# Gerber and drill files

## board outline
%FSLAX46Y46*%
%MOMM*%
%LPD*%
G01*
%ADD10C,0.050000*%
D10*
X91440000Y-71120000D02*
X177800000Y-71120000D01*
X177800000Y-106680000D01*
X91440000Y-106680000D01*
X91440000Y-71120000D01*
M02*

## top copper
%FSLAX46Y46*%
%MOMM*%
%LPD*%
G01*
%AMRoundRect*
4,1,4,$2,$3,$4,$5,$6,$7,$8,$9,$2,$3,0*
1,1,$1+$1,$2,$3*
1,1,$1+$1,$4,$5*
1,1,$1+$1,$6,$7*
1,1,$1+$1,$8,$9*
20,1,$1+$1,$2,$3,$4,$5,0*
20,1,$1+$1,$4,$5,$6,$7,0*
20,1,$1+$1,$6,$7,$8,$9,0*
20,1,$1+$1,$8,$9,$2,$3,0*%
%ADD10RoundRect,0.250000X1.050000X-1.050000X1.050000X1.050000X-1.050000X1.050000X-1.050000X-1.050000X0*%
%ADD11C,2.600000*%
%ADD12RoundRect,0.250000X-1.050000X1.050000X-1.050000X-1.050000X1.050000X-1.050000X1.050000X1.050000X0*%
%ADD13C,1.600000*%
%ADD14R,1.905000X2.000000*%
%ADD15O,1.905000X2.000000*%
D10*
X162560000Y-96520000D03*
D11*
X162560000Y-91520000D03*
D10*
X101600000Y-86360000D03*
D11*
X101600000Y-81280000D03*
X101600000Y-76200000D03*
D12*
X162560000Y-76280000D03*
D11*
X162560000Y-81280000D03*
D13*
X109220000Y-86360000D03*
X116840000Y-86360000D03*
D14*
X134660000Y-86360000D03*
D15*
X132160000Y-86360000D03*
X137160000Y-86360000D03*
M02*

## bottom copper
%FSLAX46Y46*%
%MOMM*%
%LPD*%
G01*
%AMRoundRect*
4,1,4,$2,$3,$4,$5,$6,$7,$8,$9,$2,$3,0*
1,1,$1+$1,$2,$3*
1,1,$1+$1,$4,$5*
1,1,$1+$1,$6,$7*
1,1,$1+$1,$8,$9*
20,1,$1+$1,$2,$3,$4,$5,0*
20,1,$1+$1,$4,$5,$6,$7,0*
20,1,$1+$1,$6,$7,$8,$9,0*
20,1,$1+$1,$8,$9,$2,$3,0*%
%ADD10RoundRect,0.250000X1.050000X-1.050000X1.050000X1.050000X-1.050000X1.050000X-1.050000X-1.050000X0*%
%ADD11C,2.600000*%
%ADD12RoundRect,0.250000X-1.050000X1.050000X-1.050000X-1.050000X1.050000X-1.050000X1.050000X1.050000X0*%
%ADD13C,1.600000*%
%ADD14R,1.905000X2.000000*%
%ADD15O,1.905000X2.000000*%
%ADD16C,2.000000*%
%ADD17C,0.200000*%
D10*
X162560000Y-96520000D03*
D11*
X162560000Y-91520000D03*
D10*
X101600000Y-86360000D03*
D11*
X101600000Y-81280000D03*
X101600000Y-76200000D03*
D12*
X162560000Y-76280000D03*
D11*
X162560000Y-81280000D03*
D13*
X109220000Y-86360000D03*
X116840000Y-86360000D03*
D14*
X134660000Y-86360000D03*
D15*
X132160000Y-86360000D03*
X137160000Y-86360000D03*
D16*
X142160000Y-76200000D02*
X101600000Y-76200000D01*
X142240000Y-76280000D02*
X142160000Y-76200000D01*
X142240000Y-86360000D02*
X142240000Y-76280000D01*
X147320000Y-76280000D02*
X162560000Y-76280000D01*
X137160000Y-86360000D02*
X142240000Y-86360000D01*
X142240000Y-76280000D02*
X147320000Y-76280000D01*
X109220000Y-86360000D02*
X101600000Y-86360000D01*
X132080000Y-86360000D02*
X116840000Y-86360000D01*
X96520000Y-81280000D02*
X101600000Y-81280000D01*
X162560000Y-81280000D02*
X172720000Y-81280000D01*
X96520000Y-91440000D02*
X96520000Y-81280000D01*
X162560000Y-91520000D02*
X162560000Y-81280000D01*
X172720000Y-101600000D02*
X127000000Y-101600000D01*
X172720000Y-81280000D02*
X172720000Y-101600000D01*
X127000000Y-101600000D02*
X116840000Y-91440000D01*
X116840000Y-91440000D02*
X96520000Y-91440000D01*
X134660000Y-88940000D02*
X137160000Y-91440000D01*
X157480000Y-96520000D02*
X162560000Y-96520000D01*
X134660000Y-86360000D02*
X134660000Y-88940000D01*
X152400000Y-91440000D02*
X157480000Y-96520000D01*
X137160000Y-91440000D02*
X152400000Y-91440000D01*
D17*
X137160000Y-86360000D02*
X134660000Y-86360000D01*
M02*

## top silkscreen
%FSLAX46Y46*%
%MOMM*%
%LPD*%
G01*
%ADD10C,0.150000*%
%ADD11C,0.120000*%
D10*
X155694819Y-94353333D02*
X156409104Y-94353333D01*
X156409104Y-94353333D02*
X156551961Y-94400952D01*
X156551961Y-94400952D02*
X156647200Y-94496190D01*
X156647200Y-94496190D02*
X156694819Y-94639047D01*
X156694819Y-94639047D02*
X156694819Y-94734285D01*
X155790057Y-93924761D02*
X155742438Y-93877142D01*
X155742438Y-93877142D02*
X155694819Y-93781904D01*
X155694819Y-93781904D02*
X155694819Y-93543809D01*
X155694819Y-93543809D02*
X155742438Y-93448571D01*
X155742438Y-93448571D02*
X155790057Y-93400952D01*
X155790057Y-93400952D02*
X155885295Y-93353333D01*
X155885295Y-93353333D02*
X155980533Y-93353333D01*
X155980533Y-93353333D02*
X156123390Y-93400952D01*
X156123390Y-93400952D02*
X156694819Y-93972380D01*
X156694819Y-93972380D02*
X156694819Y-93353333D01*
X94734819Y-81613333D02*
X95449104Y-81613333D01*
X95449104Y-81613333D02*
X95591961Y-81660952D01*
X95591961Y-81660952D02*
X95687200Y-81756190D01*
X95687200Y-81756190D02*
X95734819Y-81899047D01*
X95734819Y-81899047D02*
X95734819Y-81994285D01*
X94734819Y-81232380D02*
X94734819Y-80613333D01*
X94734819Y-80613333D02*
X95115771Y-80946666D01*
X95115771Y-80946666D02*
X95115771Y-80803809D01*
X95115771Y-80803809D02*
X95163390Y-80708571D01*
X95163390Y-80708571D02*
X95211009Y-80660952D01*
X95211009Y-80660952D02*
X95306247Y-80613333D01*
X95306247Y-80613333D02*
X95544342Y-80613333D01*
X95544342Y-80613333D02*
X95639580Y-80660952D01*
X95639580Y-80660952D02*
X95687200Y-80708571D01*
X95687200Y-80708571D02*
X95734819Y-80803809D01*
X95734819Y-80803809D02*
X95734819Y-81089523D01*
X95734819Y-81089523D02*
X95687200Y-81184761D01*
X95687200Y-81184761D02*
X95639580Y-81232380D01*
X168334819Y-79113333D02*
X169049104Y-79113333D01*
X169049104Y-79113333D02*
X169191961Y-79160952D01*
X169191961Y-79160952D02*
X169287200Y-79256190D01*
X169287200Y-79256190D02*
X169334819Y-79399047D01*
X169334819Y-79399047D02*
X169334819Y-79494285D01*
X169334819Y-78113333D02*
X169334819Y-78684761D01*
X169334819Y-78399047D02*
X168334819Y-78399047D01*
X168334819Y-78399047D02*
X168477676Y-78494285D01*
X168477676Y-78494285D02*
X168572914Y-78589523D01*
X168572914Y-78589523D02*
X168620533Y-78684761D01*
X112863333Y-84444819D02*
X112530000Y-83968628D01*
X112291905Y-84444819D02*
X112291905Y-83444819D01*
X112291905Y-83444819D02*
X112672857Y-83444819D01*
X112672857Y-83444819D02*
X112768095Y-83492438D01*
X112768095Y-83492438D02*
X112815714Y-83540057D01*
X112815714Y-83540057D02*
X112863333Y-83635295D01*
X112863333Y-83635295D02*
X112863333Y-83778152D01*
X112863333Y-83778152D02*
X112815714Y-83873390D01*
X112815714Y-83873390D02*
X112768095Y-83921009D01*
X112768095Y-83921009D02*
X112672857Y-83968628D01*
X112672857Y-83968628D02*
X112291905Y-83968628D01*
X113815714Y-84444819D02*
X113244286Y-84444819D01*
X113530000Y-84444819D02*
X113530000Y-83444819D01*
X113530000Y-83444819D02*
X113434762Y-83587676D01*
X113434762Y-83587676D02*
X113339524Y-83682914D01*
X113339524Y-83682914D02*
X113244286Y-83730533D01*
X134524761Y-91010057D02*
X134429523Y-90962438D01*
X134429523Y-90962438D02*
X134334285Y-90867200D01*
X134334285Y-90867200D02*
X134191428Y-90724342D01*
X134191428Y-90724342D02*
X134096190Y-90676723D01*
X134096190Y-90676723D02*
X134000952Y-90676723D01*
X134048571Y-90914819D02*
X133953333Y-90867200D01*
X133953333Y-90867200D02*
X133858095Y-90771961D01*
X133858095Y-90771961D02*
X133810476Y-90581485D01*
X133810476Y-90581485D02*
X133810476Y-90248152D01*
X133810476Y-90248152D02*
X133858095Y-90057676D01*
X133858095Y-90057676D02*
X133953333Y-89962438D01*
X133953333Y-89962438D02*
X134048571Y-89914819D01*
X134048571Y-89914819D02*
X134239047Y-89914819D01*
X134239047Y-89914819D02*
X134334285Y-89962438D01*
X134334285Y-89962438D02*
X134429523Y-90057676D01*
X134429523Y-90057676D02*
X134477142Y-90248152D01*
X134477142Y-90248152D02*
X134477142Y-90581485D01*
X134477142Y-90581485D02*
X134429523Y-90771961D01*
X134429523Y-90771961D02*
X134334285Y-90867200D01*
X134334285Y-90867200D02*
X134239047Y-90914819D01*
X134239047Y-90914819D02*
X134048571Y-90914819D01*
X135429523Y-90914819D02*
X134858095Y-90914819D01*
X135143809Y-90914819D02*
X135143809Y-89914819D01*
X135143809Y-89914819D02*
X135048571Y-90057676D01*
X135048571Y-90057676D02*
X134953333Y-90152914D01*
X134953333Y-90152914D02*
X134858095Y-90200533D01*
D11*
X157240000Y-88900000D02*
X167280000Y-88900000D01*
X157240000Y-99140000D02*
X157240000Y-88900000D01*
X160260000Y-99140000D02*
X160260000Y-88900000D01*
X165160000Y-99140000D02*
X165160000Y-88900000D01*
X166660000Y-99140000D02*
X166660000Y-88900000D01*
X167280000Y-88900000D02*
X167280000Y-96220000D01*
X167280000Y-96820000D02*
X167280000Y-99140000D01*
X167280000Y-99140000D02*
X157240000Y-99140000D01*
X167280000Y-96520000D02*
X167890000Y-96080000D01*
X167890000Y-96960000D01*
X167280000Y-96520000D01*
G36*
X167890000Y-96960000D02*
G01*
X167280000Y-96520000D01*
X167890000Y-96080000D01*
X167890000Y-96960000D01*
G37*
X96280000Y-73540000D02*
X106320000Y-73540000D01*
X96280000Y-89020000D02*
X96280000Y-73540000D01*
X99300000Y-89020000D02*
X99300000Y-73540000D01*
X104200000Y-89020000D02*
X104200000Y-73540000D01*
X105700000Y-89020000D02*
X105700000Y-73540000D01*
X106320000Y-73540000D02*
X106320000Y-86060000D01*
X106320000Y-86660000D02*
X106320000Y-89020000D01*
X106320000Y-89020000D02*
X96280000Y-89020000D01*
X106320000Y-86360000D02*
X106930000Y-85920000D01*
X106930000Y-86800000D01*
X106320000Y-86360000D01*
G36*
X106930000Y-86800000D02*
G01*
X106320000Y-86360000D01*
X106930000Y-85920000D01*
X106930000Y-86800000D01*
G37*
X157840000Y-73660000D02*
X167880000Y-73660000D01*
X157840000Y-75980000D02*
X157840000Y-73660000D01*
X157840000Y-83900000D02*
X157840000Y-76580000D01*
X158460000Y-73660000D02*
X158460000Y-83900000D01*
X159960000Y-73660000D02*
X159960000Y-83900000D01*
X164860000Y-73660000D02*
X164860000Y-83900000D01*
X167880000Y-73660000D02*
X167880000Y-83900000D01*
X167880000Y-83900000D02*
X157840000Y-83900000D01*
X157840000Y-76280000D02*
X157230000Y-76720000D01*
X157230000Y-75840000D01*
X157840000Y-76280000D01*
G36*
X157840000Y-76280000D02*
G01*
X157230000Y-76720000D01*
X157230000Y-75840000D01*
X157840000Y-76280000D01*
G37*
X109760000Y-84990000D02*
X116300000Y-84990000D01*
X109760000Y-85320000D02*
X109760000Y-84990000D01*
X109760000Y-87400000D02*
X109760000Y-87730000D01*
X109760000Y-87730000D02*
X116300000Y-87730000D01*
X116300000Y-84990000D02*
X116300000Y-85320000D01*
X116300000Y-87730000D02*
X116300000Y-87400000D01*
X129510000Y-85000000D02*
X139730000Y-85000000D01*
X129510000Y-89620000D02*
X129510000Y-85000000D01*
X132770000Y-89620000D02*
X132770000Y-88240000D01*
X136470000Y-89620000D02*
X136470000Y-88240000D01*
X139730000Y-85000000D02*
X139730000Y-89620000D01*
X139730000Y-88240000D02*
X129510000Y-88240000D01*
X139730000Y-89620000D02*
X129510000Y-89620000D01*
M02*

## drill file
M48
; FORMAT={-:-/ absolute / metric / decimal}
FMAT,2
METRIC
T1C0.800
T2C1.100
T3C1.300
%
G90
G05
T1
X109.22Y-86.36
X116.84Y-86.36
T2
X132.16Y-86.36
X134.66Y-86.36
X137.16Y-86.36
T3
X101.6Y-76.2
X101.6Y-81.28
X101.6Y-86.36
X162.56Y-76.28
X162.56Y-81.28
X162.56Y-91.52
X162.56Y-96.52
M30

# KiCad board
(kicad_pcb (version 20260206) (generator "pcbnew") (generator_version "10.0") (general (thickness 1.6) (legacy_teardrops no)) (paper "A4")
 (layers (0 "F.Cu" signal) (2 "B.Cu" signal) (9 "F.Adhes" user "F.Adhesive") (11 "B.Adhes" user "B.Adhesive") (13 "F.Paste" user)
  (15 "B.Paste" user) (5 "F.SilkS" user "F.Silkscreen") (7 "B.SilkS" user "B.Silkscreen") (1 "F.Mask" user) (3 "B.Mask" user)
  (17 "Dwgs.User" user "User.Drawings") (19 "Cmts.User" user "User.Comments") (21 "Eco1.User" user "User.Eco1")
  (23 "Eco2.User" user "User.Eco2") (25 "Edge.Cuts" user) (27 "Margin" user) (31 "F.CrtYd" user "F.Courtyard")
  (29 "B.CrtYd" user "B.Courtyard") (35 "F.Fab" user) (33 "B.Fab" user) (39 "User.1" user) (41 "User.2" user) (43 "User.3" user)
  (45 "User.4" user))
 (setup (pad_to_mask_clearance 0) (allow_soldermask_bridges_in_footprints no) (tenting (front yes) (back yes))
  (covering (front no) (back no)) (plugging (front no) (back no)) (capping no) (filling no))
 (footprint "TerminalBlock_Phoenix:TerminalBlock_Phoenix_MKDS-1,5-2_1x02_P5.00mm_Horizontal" (layer "F.Cu") (at 162.56 96.52 90)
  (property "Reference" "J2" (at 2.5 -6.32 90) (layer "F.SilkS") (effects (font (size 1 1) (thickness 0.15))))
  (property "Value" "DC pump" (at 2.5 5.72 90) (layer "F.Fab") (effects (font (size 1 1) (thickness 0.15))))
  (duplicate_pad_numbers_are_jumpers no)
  (fp_line (start 7.62 -5.32) (end 7.62 4.72) (stroke (width 0.12) (type solid)) (layer "F.SilkS"))
  (fp_line (start -2.62 -5.32) (end 7.62 -5.32) (stroke (width 0.12) (type solid)) (layer "F.SilkS"))
  (fp_line (start -2.62 -2.3) (end 7.62 -2.3) (stroke (width 0.12) (type solid)) (layer "F.SilkS"))
  (fp_line (start -2.62 2.6) (end 7.62 2.6) (stroke (width 0.12) (type solid)) (layer "F.SilkS"))
  (fp_line (start -2.62 4.1) (end 7.62 4.1) (stroke (width 0.12) (type solid)) (layer "F.SilkS"))
  (fp_line (start 7.62 4.72) (end 0.3 4.72) (stroke (width 0.12) (type solid)) (layer "F.SilkS"))
  (fp_line (start -0.3 4.72) (end -2.62 4.72) (stroke (width 0.12) (type solid)) (layer "F.SilkS"))
  (fp_line (start -2.62 4.72) (end -2.62 -5.32) (stroke (width 0.12) (type solid)) (layer "F.SilkS"))
  (fp_poly (pts (xy 0 4.72) (xy 0.44 5.33) (xy -0.44 5.33)) (stroke (width 0.12) (type solid)) (fill yes) (layer "F.SilkS"))
  (pad "1" thru_hole roundrect (at 0 0 90) (size 2.6 2.6) (drill 1.3) (layers "*.Cu" "*.Mask") (remove_unused_layers no)
   (roundrect_rratio 0.096154) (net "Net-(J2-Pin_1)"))
  (pad "2" thru_hole circle (at 5 0 90) (size 2.6 2.6) (drill 1.3) (layers "*.Cu" "*.Mask") (remove_unused_layers no) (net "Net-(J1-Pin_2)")))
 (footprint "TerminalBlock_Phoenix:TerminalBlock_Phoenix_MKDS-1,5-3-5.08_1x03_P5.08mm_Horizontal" (layer "F.Cu") (at 101.6 86.36 90)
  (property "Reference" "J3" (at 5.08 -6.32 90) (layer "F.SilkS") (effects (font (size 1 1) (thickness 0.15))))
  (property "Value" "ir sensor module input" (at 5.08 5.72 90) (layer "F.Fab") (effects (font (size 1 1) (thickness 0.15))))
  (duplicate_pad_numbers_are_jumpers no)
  (fp_line (start 12.82 -5.32) (end 12.82 4.72) (stroke (width 0.12) (type solid)) (layer "F.SilkS"))
  (fp_line (start -2.66 -5.32) (end 12.82 -5.32) (stroke (width 0.12) (type solid)) (layer "F.SilkS"))
  (fp_line (start -2.66 -2.3) (end 12.82 -2.3) (stroke (width 0.12) (type solid)) (layer "F.SilkS"))
  (fp_line (start -2.66 2.6) (end 12.82 2.6) (stroke (width 0.12) (type solid)) (layer "F.SilkS"))
  (fp_line (start -2.66 4.1) (end 12.82 4.1) (stroke (width 0.12) (type solid)) (layer "F.SilkS"))
  (fp_line (start 12.82 4.72) (end 0.3 4.72) (stroke (width 0.12) (type solid)) (layer "F.SilkS"))
  (fp_line (start -0.3 4.72) (end -2.66 4.72) (stroke (width 0.12) (type solid)) (layer "F.SilkS"))
  (fp_line (start -2.66 4.72) (end -2.66 -5.32) (stroke (width 0.12) (type solid)) (layer "F.SilkS"))
  (fp_poly (pts (xy 0 4.72) (xy 0.44 5.33) (xy -0.44 5.33)) (stroke (width 0.12) (type solid)) (fill yes) (layer "F.SilkS"))
  (pad "1" thru_hole roundrect (at 0 0 90) (size 2.6 2.6) (drill 1.3) (layers "*.Cu" "*.Mask") (remove_unused_layers no)
   (roundrect_rratio 0.096154) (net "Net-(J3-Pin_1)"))
  (pad "2" thru_hole circle (at 5.08 0 90) (size 2.6 2.6) (drill 1.3) (layers "*.Cu" "*.Mask") (remove_unused_layers no)
   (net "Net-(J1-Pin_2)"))
  (pad "3" thru_hole circle (at 10.16 0 90) (size 2.6 2.6) (drill 1.3) (layers "*.Cu" "*.Mask") (remove_unused_layers no)
   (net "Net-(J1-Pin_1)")))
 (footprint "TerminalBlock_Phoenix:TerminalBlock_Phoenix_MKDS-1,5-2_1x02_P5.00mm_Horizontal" (layer "F.Cu") (at 162.56 76.28 -90)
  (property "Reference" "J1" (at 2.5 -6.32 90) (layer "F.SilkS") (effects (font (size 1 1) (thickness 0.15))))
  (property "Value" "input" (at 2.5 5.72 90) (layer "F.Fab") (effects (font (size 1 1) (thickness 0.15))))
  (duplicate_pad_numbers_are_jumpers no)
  (fp_line (start -2.62 4.72) (end -2.62 -5.32) (stroke (width 0.12) (type solid)) (layer "F.SilkS"))
  (fp_line (start -0.3 4.72) (end -2.62 4.72) (stroke (width 0.12) (type solid)) (layer "F.SilkS"))
  (fp_line (start 7.62 4.72) (end 0.3 4.72) (stroke (width 0.12) (type solid)) (layer "F.SilkS"))
  (fp_line (start -2.62 4.1) (end 7.62 4.1) (stroke (width 0.12) (type solid)) (layer "F.SilkS"))
  (fp_line (start -2.62 2.6) (end 7.62 2.6) (stroke (width 0.12) (type solid)) (layer "F.SilkS"))
  (fp_line (start -2.62 -2.3) (end 7.62 -2.3) (stroke (width 0.12) (type solid)) (layer "F.SilkS"))
  (fp_line (start -2.62 -5.32) (end 7.62 -5.32) (stroke (width 0.12) (type solid)) (layer "F.SilkS"))
  (fp_line (start 7.62 -5.32) (end 7.62 4.72) (stroke (width 0.12) (type solid)) (layer "F.SilkS"))
  (fp_poly (pts (xy 0 4.72) (xy 0.44 5.33) (xy -0.44 5.33)) (stroke (width 0.12) (type solid)) (fill yes) (layer "F.SilkS"))
  (pad "1" thru_hole roundrect (at 0 0 270) (size 2.6 2.6) (drill 1.3) (layers "*.Cu" "*.Mask") (remove_unused_layers no)
   (roundrect_rratio 0.096154) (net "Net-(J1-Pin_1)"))
  (pad "2" thru_hole circle (at 5 0 270) (size 2.6 2.6) (drill 1.3) (layers "*.Cu" "*.Mask") (remove_unused_layers no)
   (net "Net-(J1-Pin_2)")))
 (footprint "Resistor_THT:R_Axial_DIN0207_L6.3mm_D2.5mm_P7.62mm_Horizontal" (layer "F.Cu") (at 109.22 86.36)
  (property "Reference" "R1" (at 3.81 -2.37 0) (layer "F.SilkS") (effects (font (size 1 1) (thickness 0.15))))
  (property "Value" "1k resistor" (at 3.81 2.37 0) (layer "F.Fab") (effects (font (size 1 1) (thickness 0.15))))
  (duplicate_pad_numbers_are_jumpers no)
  (fp_line (start 0.54 -1.37) (end 7.08 -1.37) (stroke (width 0.12) (type solid)) (layer "F.SilkS"))
  (fp_line (start 0.54 -1.04) (end 0.54 -1.37) (stroke (width 0.12) (type solid)) (layer "F.SilkS"))
  (fp_line (start 0.54 1.04) (end 0.54 1.37) (stroke (width 0.12) (type solid)) (layer "F.SilkS"))
  (fp_line (start 0.54 1.37) (end 7.08 1.37) (stroke (width 0.12) (type solid)) (layer "F.SilkS"))
  (fp_line (start 7.08 -1.37) (end 7.08 -1.04) (stroke (width 0.12) (type solid)) (layer "F.SilkS"))
  (fp_line (start 7.08 1.37) (end 7.08 1.04) (stroke (width 0.12) (type solid)) (layer "F.SilkS"))
  (pad "1" thru_hole circle (at 0 0) (size 1.6 1.6) (drill 0.8) (layers "*.Cu" "*.Mask") (remove_unused_layers no) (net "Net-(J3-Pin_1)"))
  (pad "2" thru_hole circle (at 7.62 0) (size 1.6 1.6) (drill 0.8) (layers "*.Cu" "*.Mask") (remove_unused_layers no) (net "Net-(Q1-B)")))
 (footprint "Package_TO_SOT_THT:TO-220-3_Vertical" (layer "F.Cu") (at 137.16 86.36 180)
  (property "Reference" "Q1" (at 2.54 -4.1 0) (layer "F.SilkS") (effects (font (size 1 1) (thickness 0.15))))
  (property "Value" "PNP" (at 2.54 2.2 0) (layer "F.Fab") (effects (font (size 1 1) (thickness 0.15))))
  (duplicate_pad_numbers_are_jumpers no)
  (fp_line (start 7.65 1.36) (end -2.57 1.36) (stroke (width 0.12) (type solid)) (layer "F.SilkS"))
  (fp_line (start 7.65 -3.26) (end 7.65 1.36) (stroke (width 0.12) (type solid)) (layer "F.SilkS"))
  (fp_line (start 4.39 -3.26) (end 4.39 -1.88) (stroke (width 0.12) (type solid)) (layer "F.SilkS"))
  (fp_line (start 0.69 -3.26) (end 0.69 -1.88) (stroke (width 0.12) (type solid)) (layer "F.SilkS"))
  (fp_line (start -2.57 1.36) (end -2.57 -3.26) (stroke (width 0.12) (type solid)) (layer "F.SilkS"))
  (fp_line (start -2.57 -1.88) (end 7.65 -1.88) (stroke (width 0.12) (type solid)) (layer "F.SilkS"))
  (fp_line (start -2.57 -3.26) (end 7.65 -3.26) (stroke (width 0.12) (type solid)) (layer "F.SilkS"))
  (pad "1" thru_hole rect (at 2.5 0 180) (size 1.905 2) (drill 1.1) (layers "*.Cu" "*.Mask") (remove_unused_layers no)
   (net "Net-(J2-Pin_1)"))
  (pad "2" thru_hole oval (at 5 0 180) (size 1.905 2) (drill 1.1) (layers "*.Cu" "*.Mask") (remove_unused_layers no) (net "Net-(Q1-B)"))
  (pad "3" thru_hole oval (at 0 0 180) (size 1.905 2) (drill 1.1) (layers "*.Cu" "*.Mask") (remove_unused_layers no) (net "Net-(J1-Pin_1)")))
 (gr_rect (start 91.44 71.12) (end 177.8 106.68) (stroke (width 0.05) (type default)) (fill no) (layer "Edge.Cuts"))
 (segment (start 142.16 76.2) (end 101.6 76.2) (width 2) (layer "B.Cu") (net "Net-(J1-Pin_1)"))
 (segment (start 142.24 76.28) (end 142.16 76.2) (width 2) (layer "B.Cu") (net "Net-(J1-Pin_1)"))
 (segment (start 142.24 86.36) (end 142.24 76.28) (width 2) (layer "B.Cu") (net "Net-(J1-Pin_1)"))
 (segment (start 147.32 76.28) (end 162.56 76.28) (width 2) (layer "B.Cu") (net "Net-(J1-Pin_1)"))
 (segment (start 137.16 86.36) (end 142.24 86.36) (width 2) (layer "B.Cu") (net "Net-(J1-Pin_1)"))
 (segment (start 142.24 76.28) (end 147.32 76.28) (width 2) (layer "B.Cu") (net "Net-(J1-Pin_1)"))
 (segment (start 109.22 86.36) (end 101.6 86.36) (width 2) (layer "B.Cu") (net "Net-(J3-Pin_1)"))
 (segment (start 132.08 86.36) (end 116.84 86.36) (width 2) (layer "B.Cu") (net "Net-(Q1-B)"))
 (segment (start 96.52 81.28) (end 101.6 81.28) (width 2) (layer "B.Cu") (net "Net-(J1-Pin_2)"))
 (segment (start 162.56 81.28) (end 172.72 81.28) (width 2) (layer "B.Cu") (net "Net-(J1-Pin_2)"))
 (segment (start 96.52 91.44) (end 96.52 81.28) (width 2) (layer "B.Cu") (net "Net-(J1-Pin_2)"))
 (segment (start 162.56 91.52) (end 162.56 81.28) (width 2) (layer "B.Cu") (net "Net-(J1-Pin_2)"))
 (segment (start 172.72 101.6) (end 127 101.6) (width 2) (layer "B.Cu") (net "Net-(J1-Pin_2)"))
 (segment (start 172.72 81.28) (end 172.72 101.6) (width 2) (layer "B.Cu") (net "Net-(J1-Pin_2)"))
 (segment (start 127 101.6) (end 116.84 91.44) (width 2) (layer "B.Cu") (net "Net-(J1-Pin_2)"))
 (segment (start 116.84 91.44) (end 96.52 91.44) (width 2) (layer "B.Cu") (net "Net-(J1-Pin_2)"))
 (segment (start 134.66 88.94) (end 137.16 91.44) (width 2) (layer "B.Cu") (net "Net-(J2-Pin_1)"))
 (segment (start 157.48 96.52) (end 162.56 96.52) (width 2) (layer "B.Cu") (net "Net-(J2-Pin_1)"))
 (segment (start 134.66 86.36) (end 134.66 88.94) (width 2) (layer "B.Cu") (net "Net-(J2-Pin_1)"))
 (segment (start 152.4 91.44) (end 157.48 96.52) (width 2) (layer "B.Cu") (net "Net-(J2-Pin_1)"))
 (segment (start 137.16 91.44) (end 152.4 91.44) (width 2) (layer "B.Cu") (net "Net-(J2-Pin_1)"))
 (segment (start 137.16 86.36) (end 134.66 86.36) (width 0.2) (layer "B.Cu") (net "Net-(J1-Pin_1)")))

